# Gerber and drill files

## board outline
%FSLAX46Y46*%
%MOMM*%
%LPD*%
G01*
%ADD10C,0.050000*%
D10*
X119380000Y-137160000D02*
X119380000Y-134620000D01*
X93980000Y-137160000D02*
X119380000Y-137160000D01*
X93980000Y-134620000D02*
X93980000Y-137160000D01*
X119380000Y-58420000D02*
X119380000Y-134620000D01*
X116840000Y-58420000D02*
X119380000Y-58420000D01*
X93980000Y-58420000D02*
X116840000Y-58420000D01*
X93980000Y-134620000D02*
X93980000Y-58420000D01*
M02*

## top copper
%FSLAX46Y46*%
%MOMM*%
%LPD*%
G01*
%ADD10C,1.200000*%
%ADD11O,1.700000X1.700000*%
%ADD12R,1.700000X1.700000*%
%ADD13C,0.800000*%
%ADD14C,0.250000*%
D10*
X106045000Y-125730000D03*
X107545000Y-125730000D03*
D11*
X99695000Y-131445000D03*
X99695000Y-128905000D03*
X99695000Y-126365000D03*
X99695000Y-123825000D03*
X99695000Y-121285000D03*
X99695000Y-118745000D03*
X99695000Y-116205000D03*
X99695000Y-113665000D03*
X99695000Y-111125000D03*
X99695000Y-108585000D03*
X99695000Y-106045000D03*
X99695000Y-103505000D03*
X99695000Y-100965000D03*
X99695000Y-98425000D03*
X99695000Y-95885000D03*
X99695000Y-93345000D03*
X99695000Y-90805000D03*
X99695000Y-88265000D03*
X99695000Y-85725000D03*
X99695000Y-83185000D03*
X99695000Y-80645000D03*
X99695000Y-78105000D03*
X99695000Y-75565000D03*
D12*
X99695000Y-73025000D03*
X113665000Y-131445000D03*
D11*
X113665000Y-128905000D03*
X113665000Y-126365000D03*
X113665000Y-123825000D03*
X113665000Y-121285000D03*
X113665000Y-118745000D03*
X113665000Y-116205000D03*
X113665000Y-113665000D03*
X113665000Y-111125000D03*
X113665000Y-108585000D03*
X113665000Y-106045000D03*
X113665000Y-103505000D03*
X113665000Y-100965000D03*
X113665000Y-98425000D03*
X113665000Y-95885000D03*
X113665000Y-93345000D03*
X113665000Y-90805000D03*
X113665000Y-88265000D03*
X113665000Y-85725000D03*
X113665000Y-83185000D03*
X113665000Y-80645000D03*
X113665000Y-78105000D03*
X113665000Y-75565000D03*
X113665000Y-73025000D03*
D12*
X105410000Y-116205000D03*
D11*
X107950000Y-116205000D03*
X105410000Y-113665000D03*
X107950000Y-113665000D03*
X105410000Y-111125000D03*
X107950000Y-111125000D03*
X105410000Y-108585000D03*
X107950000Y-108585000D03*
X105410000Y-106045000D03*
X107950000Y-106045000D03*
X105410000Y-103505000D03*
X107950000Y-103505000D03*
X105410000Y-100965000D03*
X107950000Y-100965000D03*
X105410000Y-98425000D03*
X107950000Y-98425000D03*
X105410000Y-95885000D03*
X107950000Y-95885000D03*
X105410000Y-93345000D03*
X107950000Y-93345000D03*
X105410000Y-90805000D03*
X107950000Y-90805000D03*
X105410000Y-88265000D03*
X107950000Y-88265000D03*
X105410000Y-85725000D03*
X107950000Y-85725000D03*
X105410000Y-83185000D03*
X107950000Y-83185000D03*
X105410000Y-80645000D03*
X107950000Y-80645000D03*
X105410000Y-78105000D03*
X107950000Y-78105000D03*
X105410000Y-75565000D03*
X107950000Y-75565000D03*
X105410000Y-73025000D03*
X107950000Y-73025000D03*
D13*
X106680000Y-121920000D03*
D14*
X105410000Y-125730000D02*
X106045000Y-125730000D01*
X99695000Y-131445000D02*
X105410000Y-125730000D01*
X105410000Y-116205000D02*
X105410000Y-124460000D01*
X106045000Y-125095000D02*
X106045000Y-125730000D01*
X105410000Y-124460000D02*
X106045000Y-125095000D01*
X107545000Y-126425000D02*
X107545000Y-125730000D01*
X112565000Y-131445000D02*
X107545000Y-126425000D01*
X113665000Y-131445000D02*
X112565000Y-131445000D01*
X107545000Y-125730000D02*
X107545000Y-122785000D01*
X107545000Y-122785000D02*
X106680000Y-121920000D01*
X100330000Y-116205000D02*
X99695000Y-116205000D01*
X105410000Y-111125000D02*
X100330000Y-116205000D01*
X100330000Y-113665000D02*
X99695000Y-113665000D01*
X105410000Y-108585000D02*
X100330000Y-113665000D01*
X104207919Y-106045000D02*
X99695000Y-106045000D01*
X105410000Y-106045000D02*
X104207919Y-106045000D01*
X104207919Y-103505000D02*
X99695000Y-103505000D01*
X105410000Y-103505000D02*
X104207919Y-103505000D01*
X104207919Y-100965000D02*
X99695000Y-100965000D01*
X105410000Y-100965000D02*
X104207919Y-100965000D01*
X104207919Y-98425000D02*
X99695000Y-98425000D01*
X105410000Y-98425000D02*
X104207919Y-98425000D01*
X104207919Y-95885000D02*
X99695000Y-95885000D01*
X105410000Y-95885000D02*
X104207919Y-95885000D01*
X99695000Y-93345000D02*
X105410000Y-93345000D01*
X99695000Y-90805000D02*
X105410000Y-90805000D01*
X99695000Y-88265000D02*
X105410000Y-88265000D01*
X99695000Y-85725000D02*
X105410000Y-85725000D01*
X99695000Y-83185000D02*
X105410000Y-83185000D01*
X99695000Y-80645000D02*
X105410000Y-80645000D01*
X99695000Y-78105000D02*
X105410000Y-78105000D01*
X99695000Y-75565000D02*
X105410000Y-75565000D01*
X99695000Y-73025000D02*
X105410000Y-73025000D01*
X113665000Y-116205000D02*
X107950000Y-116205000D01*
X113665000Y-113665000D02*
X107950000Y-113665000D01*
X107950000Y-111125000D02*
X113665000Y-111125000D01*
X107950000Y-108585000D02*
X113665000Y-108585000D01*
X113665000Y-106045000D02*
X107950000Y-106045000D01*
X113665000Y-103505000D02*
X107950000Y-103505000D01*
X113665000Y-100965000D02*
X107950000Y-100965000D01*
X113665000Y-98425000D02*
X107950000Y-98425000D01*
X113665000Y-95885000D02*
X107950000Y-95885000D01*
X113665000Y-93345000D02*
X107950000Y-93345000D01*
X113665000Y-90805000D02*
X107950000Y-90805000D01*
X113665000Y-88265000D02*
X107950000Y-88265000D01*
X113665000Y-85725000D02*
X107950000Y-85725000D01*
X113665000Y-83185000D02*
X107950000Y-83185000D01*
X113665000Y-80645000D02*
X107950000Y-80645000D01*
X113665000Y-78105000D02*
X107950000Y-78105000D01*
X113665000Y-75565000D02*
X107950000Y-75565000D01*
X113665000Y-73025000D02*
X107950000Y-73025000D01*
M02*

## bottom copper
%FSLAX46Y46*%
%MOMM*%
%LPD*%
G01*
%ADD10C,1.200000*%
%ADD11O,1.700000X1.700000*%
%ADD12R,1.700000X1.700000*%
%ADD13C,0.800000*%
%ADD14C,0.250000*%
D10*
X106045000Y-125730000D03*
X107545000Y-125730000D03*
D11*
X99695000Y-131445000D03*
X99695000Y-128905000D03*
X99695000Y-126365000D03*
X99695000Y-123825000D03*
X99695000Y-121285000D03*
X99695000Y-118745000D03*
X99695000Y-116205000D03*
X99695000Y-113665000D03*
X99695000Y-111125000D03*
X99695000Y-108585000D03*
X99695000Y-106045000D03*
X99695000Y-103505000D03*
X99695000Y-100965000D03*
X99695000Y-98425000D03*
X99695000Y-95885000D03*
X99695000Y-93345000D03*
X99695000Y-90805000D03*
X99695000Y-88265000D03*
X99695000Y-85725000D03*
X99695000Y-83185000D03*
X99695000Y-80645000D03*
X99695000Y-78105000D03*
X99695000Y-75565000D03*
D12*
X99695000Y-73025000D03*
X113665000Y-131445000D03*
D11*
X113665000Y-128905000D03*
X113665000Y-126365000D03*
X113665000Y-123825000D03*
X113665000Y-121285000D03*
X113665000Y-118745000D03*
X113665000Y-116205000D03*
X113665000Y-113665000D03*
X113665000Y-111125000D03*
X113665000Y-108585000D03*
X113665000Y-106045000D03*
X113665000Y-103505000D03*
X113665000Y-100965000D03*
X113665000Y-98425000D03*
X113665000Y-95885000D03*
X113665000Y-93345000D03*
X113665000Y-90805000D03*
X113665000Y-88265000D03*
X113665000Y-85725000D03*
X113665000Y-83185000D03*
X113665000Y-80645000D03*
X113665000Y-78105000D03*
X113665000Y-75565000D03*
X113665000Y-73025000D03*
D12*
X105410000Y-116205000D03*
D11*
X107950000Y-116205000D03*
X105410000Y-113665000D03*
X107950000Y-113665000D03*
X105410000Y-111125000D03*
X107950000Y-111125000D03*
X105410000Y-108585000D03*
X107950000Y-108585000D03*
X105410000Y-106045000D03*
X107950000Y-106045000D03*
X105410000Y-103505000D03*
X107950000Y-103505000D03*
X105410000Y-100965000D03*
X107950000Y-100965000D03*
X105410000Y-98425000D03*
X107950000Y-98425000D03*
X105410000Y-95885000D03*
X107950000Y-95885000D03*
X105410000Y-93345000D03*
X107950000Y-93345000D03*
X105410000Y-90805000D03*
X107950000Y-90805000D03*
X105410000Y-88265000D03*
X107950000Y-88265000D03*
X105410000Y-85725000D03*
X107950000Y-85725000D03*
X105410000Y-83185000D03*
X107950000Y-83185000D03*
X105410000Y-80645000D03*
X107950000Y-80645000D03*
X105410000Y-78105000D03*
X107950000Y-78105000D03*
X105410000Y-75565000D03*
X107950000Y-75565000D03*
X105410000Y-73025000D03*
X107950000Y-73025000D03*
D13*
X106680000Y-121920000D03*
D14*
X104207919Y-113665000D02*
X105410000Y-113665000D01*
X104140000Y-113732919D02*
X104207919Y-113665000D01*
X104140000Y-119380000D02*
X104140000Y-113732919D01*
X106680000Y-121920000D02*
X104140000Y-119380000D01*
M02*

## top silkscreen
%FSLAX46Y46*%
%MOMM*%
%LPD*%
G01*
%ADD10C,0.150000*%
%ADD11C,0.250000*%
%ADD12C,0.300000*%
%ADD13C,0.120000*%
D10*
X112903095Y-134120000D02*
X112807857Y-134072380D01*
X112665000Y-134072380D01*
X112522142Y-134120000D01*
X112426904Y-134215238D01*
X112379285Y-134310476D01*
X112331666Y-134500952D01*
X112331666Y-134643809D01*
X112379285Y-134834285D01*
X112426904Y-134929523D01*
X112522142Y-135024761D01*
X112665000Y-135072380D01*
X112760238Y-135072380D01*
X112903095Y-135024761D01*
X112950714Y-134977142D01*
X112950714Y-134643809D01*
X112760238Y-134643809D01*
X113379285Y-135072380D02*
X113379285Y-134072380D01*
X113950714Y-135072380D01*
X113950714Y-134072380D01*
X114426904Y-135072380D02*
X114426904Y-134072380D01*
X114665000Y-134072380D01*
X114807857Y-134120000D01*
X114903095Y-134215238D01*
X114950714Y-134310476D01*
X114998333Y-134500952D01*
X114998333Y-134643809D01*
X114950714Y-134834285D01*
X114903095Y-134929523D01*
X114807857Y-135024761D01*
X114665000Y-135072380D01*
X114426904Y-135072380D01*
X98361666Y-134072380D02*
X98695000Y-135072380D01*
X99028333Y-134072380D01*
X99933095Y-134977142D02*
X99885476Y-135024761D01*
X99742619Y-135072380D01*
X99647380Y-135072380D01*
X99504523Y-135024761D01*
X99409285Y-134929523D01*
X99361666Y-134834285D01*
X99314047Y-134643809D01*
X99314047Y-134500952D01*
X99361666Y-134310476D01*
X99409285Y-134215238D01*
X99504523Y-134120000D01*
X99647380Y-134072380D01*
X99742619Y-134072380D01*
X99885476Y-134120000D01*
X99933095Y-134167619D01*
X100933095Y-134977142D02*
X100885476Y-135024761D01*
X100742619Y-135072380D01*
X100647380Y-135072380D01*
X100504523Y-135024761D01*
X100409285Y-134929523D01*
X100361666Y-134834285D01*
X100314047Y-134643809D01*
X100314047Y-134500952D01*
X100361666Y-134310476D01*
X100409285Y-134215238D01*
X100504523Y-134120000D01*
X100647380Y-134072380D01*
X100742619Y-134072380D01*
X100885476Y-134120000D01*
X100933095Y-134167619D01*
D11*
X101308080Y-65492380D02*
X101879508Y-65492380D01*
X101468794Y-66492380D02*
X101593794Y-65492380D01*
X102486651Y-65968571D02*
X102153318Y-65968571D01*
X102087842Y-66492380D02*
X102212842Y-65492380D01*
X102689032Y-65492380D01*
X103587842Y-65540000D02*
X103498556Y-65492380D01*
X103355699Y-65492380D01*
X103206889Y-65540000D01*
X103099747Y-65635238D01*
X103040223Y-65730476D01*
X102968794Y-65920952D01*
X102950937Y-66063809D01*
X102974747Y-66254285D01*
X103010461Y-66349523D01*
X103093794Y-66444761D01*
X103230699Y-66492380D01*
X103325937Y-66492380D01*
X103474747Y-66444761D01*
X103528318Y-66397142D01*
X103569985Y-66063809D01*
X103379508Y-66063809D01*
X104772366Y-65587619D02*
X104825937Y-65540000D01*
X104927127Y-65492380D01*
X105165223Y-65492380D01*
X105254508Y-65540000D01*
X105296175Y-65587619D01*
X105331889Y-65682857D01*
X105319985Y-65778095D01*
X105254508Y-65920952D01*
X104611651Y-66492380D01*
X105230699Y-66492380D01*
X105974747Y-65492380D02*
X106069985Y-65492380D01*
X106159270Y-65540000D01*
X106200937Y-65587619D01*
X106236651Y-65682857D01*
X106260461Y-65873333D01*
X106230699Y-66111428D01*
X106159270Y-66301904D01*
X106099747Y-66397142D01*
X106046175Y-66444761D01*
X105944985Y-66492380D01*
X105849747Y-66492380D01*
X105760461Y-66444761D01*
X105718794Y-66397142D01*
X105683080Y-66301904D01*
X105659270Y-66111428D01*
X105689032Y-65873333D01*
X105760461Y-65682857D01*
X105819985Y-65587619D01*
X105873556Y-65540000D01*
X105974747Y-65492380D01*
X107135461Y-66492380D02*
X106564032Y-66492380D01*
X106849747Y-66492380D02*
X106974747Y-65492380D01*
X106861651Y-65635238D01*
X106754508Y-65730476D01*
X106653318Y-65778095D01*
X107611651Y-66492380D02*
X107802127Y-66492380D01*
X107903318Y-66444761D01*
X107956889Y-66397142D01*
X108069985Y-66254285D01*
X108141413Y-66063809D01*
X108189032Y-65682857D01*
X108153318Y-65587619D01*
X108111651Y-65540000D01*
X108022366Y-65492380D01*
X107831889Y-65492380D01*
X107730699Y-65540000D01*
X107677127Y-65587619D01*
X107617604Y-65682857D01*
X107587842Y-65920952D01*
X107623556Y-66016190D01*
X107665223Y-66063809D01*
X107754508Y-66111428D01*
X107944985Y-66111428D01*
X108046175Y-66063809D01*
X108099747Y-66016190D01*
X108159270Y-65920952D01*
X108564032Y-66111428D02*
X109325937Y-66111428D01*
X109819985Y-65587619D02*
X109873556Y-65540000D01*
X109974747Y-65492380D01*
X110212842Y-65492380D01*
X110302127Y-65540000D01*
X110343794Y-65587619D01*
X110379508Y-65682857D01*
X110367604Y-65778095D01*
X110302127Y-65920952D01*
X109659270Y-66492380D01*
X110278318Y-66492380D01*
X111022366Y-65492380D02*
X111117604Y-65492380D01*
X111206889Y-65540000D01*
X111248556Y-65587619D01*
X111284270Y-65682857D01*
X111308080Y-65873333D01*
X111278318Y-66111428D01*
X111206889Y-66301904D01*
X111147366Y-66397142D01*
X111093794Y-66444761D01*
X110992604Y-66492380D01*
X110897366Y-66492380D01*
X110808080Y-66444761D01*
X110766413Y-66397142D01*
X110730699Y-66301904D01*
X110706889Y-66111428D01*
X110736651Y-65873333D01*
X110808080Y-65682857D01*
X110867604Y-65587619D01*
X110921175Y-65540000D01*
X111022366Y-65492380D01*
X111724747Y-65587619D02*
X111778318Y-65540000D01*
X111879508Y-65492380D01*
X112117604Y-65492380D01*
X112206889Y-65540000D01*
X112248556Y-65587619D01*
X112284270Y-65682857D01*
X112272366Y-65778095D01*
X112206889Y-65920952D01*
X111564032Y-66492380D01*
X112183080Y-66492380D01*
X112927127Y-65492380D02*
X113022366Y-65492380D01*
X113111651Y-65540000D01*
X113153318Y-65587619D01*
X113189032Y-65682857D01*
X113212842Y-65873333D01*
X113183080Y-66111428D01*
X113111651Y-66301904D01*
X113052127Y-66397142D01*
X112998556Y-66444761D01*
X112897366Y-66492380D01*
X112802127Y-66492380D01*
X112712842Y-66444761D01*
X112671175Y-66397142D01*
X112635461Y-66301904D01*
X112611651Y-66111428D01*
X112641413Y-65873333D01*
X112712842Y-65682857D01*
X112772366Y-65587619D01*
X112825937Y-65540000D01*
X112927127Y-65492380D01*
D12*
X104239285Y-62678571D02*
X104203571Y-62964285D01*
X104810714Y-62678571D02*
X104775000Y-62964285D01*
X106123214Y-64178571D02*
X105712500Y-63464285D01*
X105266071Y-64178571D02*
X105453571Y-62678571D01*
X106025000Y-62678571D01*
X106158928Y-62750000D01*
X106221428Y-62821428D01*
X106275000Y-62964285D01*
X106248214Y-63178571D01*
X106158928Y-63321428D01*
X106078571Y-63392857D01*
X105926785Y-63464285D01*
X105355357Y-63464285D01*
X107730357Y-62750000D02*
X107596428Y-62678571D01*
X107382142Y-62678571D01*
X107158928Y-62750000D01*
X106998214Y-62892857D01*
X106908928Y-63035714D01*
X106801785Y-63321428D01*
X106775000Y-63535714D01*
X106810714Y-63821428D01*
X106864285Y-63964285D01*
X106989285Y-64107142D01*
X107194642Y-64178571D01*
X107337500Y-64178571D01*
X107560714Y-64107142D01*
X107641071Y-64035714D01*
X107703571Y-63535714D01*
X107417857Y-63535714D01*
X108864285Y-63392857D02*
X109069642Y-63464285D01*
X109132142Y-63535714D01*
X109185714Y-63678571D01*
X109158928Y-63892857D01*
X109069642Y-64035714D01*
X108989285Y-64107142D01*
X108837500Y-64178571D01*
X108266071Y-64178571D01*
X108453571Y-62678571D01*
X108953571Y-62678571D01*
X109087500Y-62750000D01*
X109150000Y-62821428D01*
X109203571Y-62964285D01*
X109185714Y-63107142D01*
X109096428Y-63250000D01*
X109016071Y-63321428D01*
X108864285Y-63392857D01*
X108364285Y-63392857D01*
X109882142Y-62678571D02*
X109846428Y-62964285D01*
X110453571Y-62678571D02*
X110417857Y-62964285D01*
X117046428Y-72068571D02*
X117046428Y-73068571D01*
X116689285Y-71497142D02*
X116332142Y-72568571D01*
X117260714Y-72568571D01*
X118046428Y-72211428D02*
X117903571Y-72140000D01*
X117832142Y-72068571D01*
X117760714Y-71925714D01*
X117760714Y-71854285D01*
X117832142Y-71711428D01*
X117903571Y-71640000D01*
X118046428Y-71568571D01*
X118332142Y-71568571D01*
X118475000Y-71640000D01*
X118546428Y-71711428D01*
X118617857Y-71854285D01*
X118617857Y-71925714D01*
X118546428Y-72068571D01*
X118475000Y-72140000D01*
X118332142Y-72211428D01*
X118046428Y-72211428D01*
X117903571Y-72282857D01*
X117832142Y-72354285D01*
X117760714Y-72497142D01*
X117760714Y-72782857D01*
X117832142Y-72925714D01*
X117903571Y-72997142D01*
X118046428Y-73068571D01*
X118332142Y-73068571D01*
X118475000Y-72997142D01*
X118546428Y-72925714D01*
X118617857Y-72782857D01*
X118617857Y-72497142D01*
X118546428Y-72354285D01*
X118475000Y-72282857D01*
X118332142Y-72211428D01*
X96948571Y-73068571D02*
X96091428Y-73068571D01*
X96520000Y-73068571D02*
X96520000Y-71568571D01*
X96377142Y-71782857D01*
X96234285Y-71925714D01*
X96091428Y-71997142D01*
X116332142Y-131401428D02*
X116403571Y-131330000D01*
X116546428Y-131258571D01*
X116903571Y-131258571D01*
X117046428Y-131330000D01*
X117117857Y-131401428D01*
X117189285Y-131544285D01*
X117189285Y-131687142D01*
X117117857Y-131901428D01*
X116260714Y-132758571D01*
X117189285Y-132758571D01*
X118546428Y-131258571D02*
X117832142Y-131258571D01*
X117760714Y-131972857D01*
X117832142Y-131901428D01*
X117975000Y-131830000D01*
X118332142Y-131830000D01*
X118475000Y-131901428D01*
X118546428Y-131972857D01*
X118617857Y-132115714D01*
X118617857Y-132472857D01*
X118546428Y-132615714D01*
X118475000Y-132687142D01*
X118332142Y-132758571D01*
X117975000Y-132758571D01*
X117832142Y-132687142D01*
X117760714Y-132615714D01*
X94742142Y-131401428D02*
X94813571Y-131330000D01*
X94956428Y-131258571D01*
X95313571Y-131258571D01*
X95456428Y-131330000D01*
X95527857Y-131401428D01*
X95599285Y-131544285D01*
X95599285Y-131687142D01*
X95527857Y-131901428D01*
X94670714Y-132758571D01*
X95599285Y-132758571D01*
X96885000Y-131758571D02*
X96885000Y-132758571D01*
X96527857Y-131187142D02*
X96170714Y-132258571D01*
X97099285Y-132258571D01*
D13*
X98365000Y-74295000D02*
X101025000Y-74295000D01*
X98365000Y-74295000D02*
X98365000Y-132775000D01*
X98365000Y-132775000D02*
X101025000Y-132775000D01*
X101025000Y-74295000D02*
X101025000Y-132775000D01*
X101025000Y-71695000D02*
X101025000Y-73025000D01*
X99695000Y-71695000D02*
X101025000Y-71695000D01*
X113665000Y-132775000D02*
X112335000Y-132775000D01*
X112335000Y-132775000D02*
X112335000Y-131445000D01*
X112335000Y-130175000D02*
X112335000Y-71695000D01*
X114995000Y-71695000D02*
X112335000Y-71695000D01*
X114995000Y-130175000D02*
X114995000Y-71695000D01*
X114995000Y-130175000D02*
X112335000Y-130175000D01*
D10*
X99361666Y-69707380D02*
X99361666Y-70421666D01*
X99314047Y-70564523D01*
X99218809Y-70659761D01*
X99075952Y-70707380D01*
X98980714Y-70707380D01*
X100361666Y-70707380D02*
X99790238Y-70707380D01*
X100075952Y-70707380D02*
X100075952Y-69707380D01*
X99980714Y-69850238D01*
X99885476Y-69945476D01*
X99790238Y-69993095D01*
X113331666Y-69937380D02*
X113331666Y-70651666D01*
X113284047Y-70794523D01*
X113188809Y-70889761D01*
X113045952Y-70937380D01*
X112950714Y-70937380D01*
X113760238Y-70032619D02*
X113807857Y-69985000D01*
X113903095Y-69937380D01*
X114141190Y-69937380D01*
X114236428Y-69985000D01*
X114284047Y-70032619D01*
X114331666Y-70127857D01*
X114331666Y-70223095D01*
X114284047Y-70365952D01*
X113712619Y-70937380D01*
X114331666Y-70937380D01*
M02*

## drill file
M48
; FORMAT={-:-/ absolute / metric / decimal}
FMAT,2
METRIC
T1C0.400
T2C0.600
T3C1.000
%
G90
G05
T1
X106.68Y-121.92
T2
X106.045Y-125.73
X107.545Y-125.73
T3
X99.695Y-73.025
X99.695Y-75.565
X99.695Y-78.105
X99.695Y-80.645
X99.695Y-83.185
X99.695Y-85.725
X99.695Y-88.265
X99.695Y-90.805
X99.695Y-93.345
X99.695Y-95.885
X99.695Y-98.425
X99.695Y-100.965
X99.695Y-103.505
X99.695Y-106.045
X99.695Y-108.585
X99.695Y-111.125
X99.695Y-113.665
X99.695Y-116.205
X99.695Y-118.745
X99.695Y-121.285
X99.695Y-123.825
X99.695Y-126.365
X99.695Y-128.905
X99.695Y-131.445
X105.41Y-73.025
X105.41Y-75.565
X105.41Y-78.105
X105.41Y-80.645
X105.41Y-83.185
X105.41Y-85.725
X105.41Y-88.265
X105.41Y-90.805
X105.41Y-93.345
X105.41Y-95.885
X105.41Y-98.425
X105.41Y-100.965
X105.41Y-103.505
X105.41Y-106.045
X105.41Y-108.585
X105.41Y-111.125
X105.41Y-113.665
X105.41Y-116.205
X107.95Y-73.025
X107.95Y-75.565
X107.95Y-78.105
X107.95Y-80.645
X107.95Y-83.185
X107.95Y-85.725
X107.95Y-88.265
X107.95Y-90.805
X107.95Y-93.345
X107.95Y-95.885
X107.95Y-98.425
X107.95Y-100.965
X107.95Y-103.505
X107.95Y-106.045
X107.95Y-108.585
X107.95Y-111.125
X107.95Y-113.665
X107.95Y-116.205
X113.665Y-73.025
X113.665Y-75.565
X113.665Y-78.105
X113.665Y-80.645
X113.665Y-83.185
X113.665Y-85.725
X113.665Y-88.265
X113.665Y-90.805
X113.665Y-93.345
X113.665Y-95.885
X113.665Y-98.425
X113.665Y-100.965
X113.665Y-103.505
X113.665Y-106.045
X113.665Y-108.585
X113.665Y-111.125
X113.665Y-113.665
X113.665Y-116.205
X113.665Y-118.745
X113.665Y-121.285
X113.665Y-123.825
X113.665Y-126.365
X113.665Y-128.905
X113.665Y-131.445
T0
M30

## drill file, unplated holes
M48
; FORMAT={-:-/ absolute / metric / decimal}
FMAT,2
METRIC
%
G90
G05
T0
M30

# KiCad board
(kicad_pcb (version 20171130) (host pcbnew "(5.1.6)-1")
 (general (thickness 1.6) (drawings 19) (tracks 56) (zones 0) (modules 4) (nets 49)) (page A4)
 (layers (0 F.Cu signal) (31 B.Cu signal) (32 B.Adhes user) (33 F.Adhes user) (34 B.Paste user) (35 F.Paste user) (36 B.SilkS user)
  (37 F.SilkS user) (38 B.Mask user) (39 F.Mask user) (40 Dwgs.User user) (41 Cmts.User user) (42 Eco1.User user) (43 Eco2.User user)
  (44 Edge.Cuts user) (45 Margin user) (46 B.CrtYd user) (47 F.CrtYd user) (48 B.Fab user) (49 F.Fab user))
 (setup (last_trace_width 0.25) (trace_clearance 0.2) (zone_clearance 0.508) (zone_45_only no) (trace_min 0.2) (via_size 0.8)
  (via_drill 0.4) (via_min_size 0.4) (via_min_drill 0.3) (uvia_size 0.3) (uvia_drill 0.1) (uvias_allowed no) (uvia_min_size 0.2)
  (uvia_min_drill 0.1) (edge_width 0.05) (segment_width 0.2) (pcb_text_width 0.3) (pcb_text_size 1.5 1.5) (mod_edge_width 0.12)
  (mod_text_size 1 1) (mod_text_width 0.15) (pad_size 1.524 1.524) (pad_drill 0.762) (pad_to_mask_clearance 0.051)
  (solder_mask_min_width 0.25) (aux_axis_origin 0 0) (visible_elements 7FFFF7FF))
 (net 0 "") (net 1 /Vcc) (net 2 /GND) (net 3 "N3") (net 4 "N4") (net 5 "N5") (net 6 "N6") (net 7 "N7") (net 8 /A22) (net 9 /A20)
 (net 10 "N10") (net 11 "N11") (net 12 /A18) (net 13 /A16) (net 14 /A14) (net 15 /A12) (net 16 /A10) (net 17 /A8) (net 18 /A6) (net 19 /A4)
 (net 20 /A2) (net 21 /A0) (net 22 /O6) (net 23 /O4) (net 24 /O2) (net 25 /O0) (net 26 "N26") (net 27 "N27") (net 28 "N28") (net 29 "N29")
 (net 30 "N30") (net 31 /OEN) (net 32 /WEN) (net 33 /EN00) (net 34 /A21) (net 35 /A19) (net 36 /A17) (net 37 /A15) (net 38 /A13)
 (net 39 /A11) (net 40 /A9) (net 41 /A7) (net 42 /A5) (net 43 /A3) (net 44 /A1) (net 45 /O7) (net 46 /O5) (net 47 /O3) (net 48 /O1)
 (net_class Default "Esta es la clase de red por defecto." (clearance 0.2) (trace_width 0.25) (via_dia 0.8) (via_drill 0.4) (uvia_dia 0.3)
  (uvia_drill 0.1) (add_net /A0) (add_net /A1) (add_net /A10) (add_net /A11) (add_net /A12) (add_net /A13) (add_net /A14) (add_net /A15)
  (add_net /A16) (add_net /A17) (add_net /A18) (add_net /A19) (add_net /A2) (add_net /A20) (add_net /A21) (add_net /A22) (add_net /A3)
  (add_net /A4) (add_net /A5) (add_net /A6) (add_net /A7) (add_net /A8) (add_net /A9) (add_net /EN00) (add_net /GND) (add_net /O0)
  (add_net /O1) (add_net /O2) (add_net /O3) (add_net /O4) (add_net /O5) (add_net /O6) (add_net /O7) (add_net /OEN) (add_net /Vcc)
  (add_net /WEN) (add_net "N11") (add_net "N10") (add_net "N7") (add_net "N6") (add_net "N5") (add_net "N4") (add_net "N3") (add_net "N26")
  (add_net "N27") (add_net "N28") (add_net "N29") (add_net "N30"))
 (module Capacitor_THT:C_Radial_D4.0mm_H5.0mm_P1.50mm (layer B.Cu) (at 106.045 125.73)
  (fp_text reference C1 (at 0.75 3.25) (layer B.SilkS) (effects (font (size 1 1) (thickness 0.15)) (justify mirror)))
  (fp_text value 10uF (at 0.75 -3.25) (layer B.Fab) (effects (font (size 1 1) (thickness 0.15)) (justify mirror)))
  (pad 1 thru_hole circle (at 0 0) (size 1.2 1.2) (drill 0.6) (layers *.Cu *.Mask) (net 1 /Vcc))
  (pad 2 thru_hole circle (at 1.5 0) (size 1.2 1.2) (drill 0.6) (layers *.Cu *.Mask) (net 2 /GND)))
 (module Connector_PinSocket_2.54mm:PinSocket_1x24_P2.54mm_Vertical (layer F.Cu) (at 99.695 73.025)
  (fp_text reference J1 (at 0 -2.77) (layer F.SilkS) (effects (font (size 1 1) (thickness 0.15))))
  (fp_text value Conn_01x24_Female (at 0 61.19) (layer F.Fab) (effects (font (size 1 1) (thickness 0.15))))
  (fp_line (start -1.33 1.27) (end 1.33 1.27) (layer F.SilkS) (width 0.12))
  (fp_line (start -1.33 1.27) (end -1.33 59.75) (layer F.SilkS) (width 0.12))
  (fp_line (start -1.33 59.75) (end 1.33 59.75) (layer F.SilkS) (width 0.12))
  (fp_line (start 1.33 1.27) (end 1.33 59.75) (layer F.SilkS) (width 0.12))
  (fp_line (start 1.33 -1.33) (end 1.33 0) (layer F.SilkS) (width 0.12))
  (fp_line (start 0 -1.33) (end 1.33 -1.33) (layer F.SilkS) (width 0.12))
  (pad 24 thru_hole oval (at 0 58.42) (size 1.7 1.7) (drill 1) (layers *.Cu *.Mask) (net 1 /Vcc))
  (pad 23 thru_hole oval (at 0 55.88) (size 1.7 1.7) (drill 1) (layers *.Cu *.Mask) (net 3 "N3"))
  (pad 22 thru_hole oval (at 0 53.34) (size 1.7 1.7) (drill 1) (layers *.Cu *.Mask) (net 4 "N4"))
  (pad 21 thru_hole oval (at 0 50.8) (size 1.7 1.7) (drill 1) (layers *.Cu *.Mask) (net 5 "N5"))
  (pad 20 thru_hole oval (at 0 48.26) (size 1.7 1.7) (drill 1) (layers *.Cu *.Mask) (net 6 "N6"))
  (pad 19 thru_hole oval (at 0 45.72) (size 1.7 1.7) (drill 1) (layers *.Cu *.Mask) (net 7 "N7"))
  (pad 18 thru_hole oval (at 0 43.18) (size 1.7 1.7) (drill 1) (layers *.Cu *.Mask) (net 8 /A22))
  (pad 17 thru_hole oval (at 0 40.64) (size 1.7 1.7) (drill 1) (layers *.Cu *.Mask) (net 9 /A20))
  (pad 16 thru_hole oval (at 0 38.1) (size 1.7 1.7) (drill 1) (layers *.Cu *.Mask) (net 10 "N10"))
  (pad 15 thru_hole oval (at 0 35.56) (size 1.7 1.7) (drill 1) (layers *.Cu *.Mask) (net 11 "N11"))
  (pad 14 thru_hole oval (at 0 33.02) (size 1.7 1.7) (drill 1) (layers *.Cu *.Mask) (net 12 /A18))
  (pad 13 thru_hole oval (at 0 30.48) (size 1.7 1.7) (drill 1) (layers *.Cu *.Mask) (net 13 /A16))
  (pad 12 thru_hole oval (at 0 27.94) (size 1.7 1.7) (drill 1) (layers *.Cu *.Mask) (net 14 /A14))
  (pad 11 thru_hole oval (at 0 25.4) (size 1.7 1.7) (drill 1) (layers *.Cu *.Mask) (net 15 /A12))
  (pad 10 thru_hole oval (at 0 22.86) (size 1.7 1.7) (drill 1) (layers *.Cu *.Mask) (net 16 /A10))
  (pad 9 thru_hole oval (at 0 20.32) (size 1.7 1.7) (drill 1) (layers *.Cu *.Mask) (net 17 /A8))
  (pad 8 thru_hole oval (at 0 17.78) (size 1.7 1.7) (drill 1) (layers *.Cu *.Mask) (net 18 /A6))
  (pad 7 thru_hole oval (at 0 15.24) (size 1.7 1.7) (drill 1) (layers *.Cu *.Mask) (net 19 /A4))
  (pad 6 thru_hole oval (at 0 12.7) (size 1.7 1.7) (drill 1) (layers *.Cu *.Mask) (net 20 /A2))
  (pad 5 thru_hole oval (at 0 10.16) (size 1.7 1.7) (drill 1) (layers *.Cu *.Mask) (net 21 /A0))
  (pad 4 thru_hole oval (at 0 7.62) (size 1.7 1.7) (drill 1) (layers *.Cu *.Mask) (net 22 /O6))
  (pad 3 thru_hole oval (at 0 5.08) (size 1.7 1.7) (drill 1) (layers *.Cu *.Mask) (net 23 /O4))
  (pad 2 thru_hole oval (at 0 2.54) (size 1.7 1.7) (drill 1) (layers *.Cu *.Mask) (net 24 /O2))
  (pad 1 thru_hole rect (at 0 0) (size 1.7 1.7) (drill 1) (layers *.Cu *.Mask) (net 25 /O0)))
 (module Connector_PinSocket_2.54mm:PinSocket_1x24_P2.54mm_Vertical (layer F.Cu) (at 113.665 131.445 180)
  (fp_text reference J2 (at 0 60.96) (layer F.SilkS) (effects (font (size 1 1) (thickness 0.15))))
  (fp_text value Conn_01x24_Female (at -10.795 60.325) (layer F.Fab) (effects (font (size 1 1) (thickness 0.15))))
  (fp_line (start 0 -1.33) (end 1.33 -1.33) (layer F.SilkS) (width 0.12))
  (fp_line (start 1.33 -1.33) (end 1.33 0) (layer F.SilkS) (width 0.12))
  (fp_line (start 1.33 1.27) (end 1.33 59.75) (layer F.SilkS) (width 0.12))
  (fp_line (start -1.33 59.75) (end 1.33 59.75) (layer F.SilkS) (width 0.12))
  (fp_line (start -1.33 1.27) (end -1.33 59.75) (layer F.SilkS) (width 0.12))
  (fp_line (start -1.33 1.27) (end 1.33 1.27) (layer F.SilkS) (width 0.12))
  (pad 1 thru_hole rect (at 0 0 180) (size 1.7 1.7) (drill 1) (layers *.Cu *.Mask) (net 2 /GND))
  (pad 2 thru_hole oval (at 0 2.54 180) (size 1.7 1.7) (drill 1) (layers *.Cu *.Mask) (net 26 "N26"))
  (pad 3 thru_hole oval (at 0 5.08 180) (size 1.7 1.7) (drill 1) (layers *.Cu *.Mask) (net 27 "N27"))
  (pad 4 thru_hole oval (at 0 7.62 180) (size 1.7 1.7) (drill 1) (layers *.Cu *.Mask) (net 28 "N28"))
  (pad 5 thru_hole oval (at 0 10.16 180) (size 1.7 1.7) (drill 1) (layers *.Cu *.Mask) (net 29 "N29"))
  (pad 6 thru_hole oval (at 0 12.7 180) (size 1.7 1.7) (drill 1) (layers *.Cu *.Mask) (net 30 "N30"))
  (pad 7 thru_hole oval (at 0 15.24 180) (size 1.7 1.7) (drill 1) (layers *.Cu *.Mask) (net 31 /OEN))
  (pad 8 thru_hole oval (at 0 17.78 180) (size 1.7 1.7) (drill 1) (layers *.Cu *.Mask) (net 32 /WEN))
  (pad 9 thru_hole oval (at 0 20.32 180) (size 1.7 1.7) (drill 1) (layers *.Cu *.Mask) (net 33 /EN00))
  (pad 10 thru_hole oval (at 0 22.86 180) (size 1.7 1.7) (drill 1) (layers *.Cu *.Mask) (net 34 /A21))
  (pad 11 thru_hole oval (at 0 25.4 180) (size 1.7 1.7) (drill 1) (layers *.Cu *.Mask) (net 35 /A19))
  (pad 12 thru_hole oval (at 0 27.94 180) (size 1.7 1.7) (drill 1) (layers *.Cu *.Mask) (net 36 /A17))
  (pad 13 thru_hole oval (at 0 30.48 180) (size 1.7 1.7) (drill 1) (layers *.Cu *.Mask) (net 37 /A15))
  (pad 14 thru_hole oval (at 0 33.02 180) (size 1.7 1.7) (drill 1) (layers *.Cu *.Mask) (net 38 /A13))
  (pad 15 thru_hole oval (at 0 35.56 180) (size 1.7 1.7) (drill 1) (layers *.Cu *.Mask) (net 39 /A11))
  (pad 16 thru_hole oval (at 0 38.1 180) (size 1.7 1.7) (drill 1) (layers *.Cu *.Mask) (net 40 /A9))
  (pad 17 thru_hole oval (at 0 40.64 180) (size 1.7 1.7) (drill 1) (layers *.Cu *.Mask) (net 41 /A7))
  (pad 18 thru_hole oval (at 0 43.18 180) (size 1.7 1.7) (drill 1) (layers *.Cu *.Mask) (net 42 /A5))
  (pad 19 thru_hole oval (at 0 45.72 180) (size 1.7 1.7) (drill 1) (layers *.Cu *.Mask) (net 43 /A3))
  (pad 20 thru_hole oval (at 0 48.26 180) (size 1.7 1.7) (drill 1) (layers *.Cu *.Mask) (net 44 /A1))
  (pad 21 thru_hole oval (at 0 50.8 180) (size 1.7 1.7) (drill 1) (layers *.Cu *.Mask) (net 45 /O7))
  (pad 22 thru_hole oval (at 0 53.34 180) (size 1.7 1.7) (drill 1) (layers *.Cu *.Mask) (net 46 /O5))
  (pad 23 thru_hole oval (at 0 55.88 180) (size 1.7 1.7) (drill 1) (layers *.Cu *.Mask) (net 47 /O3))
  (pad 24 thru_hole oval (at 0 58.42 180) (size 1.7 1.7) (drill 1) (layers *.Cu *.Mask) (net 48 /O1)))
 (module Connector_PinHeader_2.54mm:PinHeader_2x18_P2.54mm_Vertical (layer B.Cu) (at 105.41 116.205)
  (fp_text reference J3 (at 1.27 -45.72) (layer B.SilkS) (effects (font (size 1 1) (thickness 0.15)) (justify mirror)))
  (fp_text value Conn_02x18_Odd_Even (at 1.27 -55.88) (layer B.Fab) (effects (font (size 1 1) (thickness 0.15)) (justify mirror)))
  (pad 1 thru_hole rect (at 0 0) (size 1.7 1.7) (drill 1) (layers *.Cu *.Mask) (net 1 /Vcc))
  (pad 2 thru_hole oval (at 2.54 0) (size 1.7 1.7) (drill 1) (layers *.Cu *.Mask) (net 31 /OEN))
  (pad 3 thru_hole oval (at 0 -2.54) (size 1.7 1.7) (drill 1) (layers *.Cu *.Mask) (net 2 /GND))
  (pad 4 thru_hole oval (at 2.54 -2.54) (size 1.7 1.7) (drill 1) (layers *.Cu *.Mask) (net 32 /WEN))
  (pad 5 thru_hole oval (at 0 -5.08) (size 1.7 1.7) (drill 1) (layers *.Cu *.Mask) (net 8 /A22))
  (pad 6 thru_hole oval (at 2.54 -5.08) (size 1.7 1.7) (drill 1) (layers *.Cu *.Mask) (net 33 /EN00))
  (pad 7 thru_hole oval (at 0 -7.62) (size 1.7 1.7) (drill 1) (layers *.Cu *.Mask) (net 9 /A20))
  (pad 8 thru_hole oval (at 2.54 -7.62) (size 1.7 1.7) (drill 1) (layers *.Cu *.Mask) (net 34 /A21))
  (pad 9 thru_hole oval (at 0 -10.16) (size 1.7 1.7) (drill 1) (layers *.Cu *.Mask) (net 12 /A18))
  (pad 10 thru_hole oval (at 2.54 -10.16) (size 1.7 1.7) (drill 1) (layers *.Cu *.Mask) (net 35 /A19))
  (pad 11 thru_hole oval (at 0 -12.7) (size 1.7 1.7) (drill 1) (layers *.Cu *.Mask) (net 13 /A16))
  (pad 12 thru_hole oval (at 2.54 -12.7) (size 1.7 1.7) (drill 1) (layers *.Cu *.Mask) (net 36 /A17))
  (pad 13 thru_hole oval (at 0 -15.24) (size 1.7 1.7) (drill 1) (layers *.Cu *.Mask) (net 14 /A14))
  (pad 14 thru_hole oval (at 2.54 -15.24) (size 1.7 1.7) (drill 1) (layers *.Cu *.Mask) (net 37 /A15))
  (pad 15 thru_hole oval (at 0 -17.78) (size 1.7 1.7) (drill 1) (layers *.Cu *.Mask) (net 15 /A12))
  (pad 16 thru_hole oval (at 2.54 -17.78) (size 1.7 1.7) (drill 1) (layers *.Cu *.Mask) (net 38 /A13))
  (pad 17 thru_hole oval (at 0 -20.32) (size 1.7 1.7) (drill 1) (layers *.Cu *.Mask) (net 16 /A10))
  (pad 18 thru_hole oval (at 2.54 -20.32) (size 1.7 1.7) (drill 1) (layers *.Cu *.Mask) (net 39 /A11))
  (pad 19 thru_hole oval (at 0 -22.86) (size 1.7 1.7) (drill 1) (layers *.Cu *.Mask) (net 17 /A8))
  (pad 20 thru_hole oval (at 2.54 -22.86) (size 1.7 1.7) (drill 1) (layers *.Cu *.Mask) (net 40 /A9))
  (pad 21 thru_hole oval (at 0 -25.4) (size 1.7 1.7) (drill 1) (layers *.Cu *.Mask) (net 18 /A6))
  (pad 22 thru_hole oval (at 2.54 -25.4) (size 1.7 1.7) (drill 1) (layers *.Cu *.Mask) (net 41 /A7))
  (pad 23 thru_hole oval (at 0 -27.94) (size 1.7 1.7) (drill 1) (layers *.Cu *.Mask) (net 19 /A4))
  (pad 24 thru_hole oval (at 2.54 -27.94) (size 1.7 1.7) (drill 1) (layers *.Cu *.Mask) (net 42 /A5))
  (pad 25 thru_hole oval (at 0 -30.48) (size 1.7 1.7) (drill 1) (layers *.Cu *.Mask) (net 20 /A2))
  (pad 26 thru_hole oval (at 2.54 -30.48) (size 1.7 1.7) (drill 1) (layers *.Cu *.Mask) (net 43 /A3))
  (pad 27 thru_hole oval (at 0 -33.02) (size 1.7 1.7) (drill 1) (layers *.Cu *.Mask) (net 21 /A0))
  (pad 28 thru_hole oval (at 2.54 -33.02) (size 1.7 1.7) (drill 1) (layers *.Cu *.Mask) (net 44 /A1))
  (pad 29 thru_hole oval (at 0 -35.56) (size 1.7 1.7) (drill 1) (layers *.Cu *.Mask) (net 22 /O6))
  (pad 30 thru_hole oval (at 2.54 -35.56) (size 1.7 1.7) (drill 1) (layers *.Cu *.Mask) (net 45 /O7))
  (pad 31 thru_hole oval (at 0 -38.1) (size 1.7 1.7) (drill 1) (layers *.Cu *.Mask) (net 23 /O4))
  (pad 32 thru_hole oval (at 2.54 -38.1) (size 1.7 1.7) (drill 1) (layers *.Cu *.Mask) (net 46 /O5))
  (pad 33 thru_hole oval (at 0 -40.64) (size 1.7 1.7) (drill 1) (layers *.Cu *.Mask) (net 24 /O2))
  (pad 34 thru_hole oval (at 2.54 -40.64) (size 1.7 1.7) (drill 1) (layers *.Cu *.Mask) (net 47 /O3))
  (pad 35 thru_hole oval (at 0 -43.18) (size 1.7 1.7) (drill 1) (layers *.Cu *.Mask) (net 25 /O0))
  (pad 36 thru_hole oval (at 2.54 -43.18) (size 1.7 1.7) (drill 1) (layers *.Cu *.Mask) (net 48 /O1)))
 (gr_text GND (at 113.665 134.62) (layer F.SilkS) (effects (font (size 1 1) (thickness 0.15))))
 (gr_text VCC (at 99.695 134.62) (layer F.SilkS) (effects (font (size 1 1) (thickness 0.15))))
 (gr_line (start 119.38 137.16) (end 119.38 134.62) (layer Edge.Cuts) (width 0.05))
 (gr_line (start 93.98 137.16) (end 119.38 137.16) (layer Edge.Cuts) (width 0.05))
 (gr_line (start 93.98 134.62) (end 93.98 137.16) (layer Edge.Cuts) (width 0.05))
 (gr_line (start 119.38 58.42) (end 119.38 134.62) (layer Edge.Cuts) (width 0.05))
 (gr_line (start 116.84 58.42) (end 119.38 58.42) (layer Edge.Cuts) (width 0.05))
 (gr_line (start 93.98 58.42) (end 116.84 58.42) (layer Edge.Cuts) (width 0.05))
 (gr_line (start 93.98 134.62) (end 93.98 58.42) (layer Edge.Cuts) (width 0.05))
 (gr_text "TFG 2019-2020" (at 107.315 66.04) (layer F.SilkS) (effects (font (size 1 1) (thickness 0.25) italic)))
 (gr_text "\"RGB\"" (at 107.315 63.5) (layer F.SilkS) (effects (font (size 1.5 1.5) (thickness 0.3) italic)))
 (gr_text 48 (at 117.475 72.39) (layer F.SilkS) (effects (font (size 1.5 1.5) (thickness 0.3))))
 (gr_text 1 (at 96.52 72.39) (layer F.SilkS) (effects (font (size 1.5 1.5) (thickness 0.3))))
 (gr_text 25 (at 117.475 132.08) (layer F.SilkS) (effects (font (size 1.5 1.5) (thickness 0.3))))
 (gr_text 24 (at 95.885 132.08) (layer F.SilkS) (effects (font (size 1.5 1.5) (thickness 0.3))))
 (segment (start 105.41 125.73) (end 106.045 125.73) (width 0.25) (layer F.Cu) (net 1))
 (segment (start 99.695 131.445) (end 105.41 125.73) (width 0.25) (layer F.Cu) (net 1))
 (segment (start 105.41 116.205) (end 105.41 124.46) (width 0.25) (layer F.Cu) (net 1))
 (segment (start 106.045 125.095) (end 106.045 125.73) (width 0.25) (layer F.Cu) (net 1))
 (segment (start 105.41 124.46) (end 106.045 125.095) (width 0.25) (layer F.Cu) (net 1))
 (segment (start 107.545 126.425) (end 107.545 125.73) (width 0.25) (layer F.Cu) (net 2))
 (segment (start 112.565 131.445) (end 107.545 126.425) (width 0.25) (layer F.Cu) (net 2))
 (segment (start 113.665 131.445) (end 112.565 131.445) (width 0.25) (layer F.Cu) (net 2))
 (segment (start 107.545 125.73) (end 107.545 122.785) (width 0.25) (layer F.Cu) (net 2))
 (segment (start 107.545 122.785) (end 106.68 121.92) (width 0.25) (layer F.Cu) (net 2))
 (via (at 106.68 121.92) (size 0.8) (drill 0.4) (layers F.Cu B.Cu) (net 2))
 (segment (start 104.207919 113.665) (end 105.41 113.665) (width 0.25) (layer B.Cu) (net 2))
 (segment (start 104.14 113.732919) (end 104.207919 113.665) (width 0.25) (layer B.Cu) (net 2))
 (segment (start 104.14 119.38) (end 104.14 113.732919) (width 0.25) (layer B.Cu) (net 2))
 (segment (start 106.68 121.92) (end 104.14 119.38) (width 0.25) (layer B.Cu) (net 2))
 (segment (start 100.33 116.205) (end 99.695 116.205) (width 0.25) (layer F.Cu) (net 8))
 (segment (start 105.41 111.125) (end 100.33 116.205) (width 0.25) (layer F.Cu) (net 8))
 (segment (start 100.33 113.665) (end 99.695 113.665) (width 0.25) (layer F.Cu) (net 9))
 (segment (start 105.41 108.585) (end 100.33 113.665) (width 0.25) (layer F.Cu) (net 9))
 (segment (start 104.207919 106.045) (end 99.695 106.045) (width 0.25) (layer F.Cu) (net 12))
 (segment (start 105.41 106.045) (end 104.207919 106.045) (width 0.25) (layer F.Cu) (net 12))
 (segment (start 104.207919 103.505) (end 99.695 103.505) (width 0.25) (layer F.Cu) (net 13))
 (segment (start 105.41 103.505) (end 104.207919 103.505) (width 0.25) (layer F.Cu) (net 13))
 (segment (start 104.207919 100.965) (end 99.695 100.965) (width 0.25) (layer F.Cu) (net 14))
 (segment (start 105.41 100.965) (end 104.207919 100.965) (width 0.25) (layer F.Cu) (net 14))
 (segment (start 104.207919 98.425) (end 99.695 98.425) (width 0.25) (layer F.Cu) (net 15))
 (segment (start 105.41 98.425) (end 104.207919 98.425) (width 0.25) (layer F.Cu) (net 15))
 (segment (start 104.207919 95.885) (end 99.695 95.885) (width 0.25) (layer F.Cu) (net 16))
 (segment (start 105.41 95.885) (end 104.207919 95.885) (width 0.25) (layer F.Cu) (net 16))
 (segment (start 99.695 93.345) (end 105.41 93.345) (width 0.25) (layer F.Cu) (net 17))
 (segment (start 99.695 90.805) (end 105.41 90.805) (width 0.25) (layer F.Cu) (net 18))
 (segment (start 99.695 88.265) (end 105.41 88.265) (width 0.25) (layer F.Cu) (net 19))
 (segment (start 99.695 85.725) (end 105.41 85.725) (width 0.25) (layer F.Cu) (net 20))
 (segment (start 99.695 83.185) (end 105.41 83.185) (width 0.25) (layer F.Cu) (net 21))
 (segment (start 99.695 80.645) (end 105.41 80.645) (width 0.25) (layer F.Cu) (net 22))
 (segment (start 99.695 78.105) (end 105.41 78.105) (width 0.25) (layer F.Cu) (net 23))
 (segment (start 99.695 75.565) (end 105.41 75.565) (width 0.25) (layer F.Cu) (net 24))
 (segment (start 99.695 73.025) (end 105.41 73.025) (width 0.25) (layer F.Cu) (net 25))
 (segment (start 113.665 116.205) (end 107.95 116.205) (width 0.25) (layer F.Cu) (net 31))
 (segment (start 113.665 113.665) (end 107.95 113.665) (width 0.25) (layer F.Cu) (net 32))
 (segment (start 107.95 111.125) (end 113.665 111.125) (width 0.25) (layer F.Cu) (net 33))
 (segment (start 107.95 108.585) (end 113.665 108.585) (width 0.25) (layer F.Cu) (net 34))
 (segment (start 113.665 106.045) (end 107.95 106.045) (width 0.25) (layer F.Cu) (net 35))
 (segment (start 113.665 103.505) (end 107.95 103.505) (width 0.25) (layer F.Cu) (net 36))
 (segment (start 113.665 100.965) (end 107.95 100.965) (width 0.25) (layer F.Cu) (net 37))
 (segment (start 113.665 98.425) (end 107.95 98.425) (width 0.25) (layer F.Cu) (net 38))
 (segment (start 113.665 95.885) (end 107.95 95.885) (width 0.25) (layer F.Cu) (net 39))
 (segment (start 113.665 93.345) (end 107.95 93.345) (width 0.25) (layer F.Cu) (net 40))
 (segment (start 113.665 90.805) (end 107.95 90.805) (width 0.25) (layer F.Cu) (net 41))
 (segment (start 113.665 88.265) (end 107.95 88.265) (width 0.25) (layer F.Cu) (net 42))
 (segment (start 113.665 85.725) (end 107.95 85.725) (width 0.25) (layer F.Cu) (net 43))
 (segment (start 113.665 83.185) (end 107.95 83.185) (width 0.25) (layer F.Cu) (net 44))
 (segment (start 113.665 80.645) (end 107.95 80.645) (width 0.25) (layer F.Cu) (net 45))
 (segment (start 113.665 78.105) (end 107.95 78.105) (width 0.25) (layer F.Cu) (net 46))
 (segment (start 113.665 75.565) (end 107.95 75.565) (width 0.25) (layer F.Cu) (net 47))
 (segment (start 113.665 73.025) (end 107.95 73.025) (width 0.25) (layer F.Cu) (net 48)))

